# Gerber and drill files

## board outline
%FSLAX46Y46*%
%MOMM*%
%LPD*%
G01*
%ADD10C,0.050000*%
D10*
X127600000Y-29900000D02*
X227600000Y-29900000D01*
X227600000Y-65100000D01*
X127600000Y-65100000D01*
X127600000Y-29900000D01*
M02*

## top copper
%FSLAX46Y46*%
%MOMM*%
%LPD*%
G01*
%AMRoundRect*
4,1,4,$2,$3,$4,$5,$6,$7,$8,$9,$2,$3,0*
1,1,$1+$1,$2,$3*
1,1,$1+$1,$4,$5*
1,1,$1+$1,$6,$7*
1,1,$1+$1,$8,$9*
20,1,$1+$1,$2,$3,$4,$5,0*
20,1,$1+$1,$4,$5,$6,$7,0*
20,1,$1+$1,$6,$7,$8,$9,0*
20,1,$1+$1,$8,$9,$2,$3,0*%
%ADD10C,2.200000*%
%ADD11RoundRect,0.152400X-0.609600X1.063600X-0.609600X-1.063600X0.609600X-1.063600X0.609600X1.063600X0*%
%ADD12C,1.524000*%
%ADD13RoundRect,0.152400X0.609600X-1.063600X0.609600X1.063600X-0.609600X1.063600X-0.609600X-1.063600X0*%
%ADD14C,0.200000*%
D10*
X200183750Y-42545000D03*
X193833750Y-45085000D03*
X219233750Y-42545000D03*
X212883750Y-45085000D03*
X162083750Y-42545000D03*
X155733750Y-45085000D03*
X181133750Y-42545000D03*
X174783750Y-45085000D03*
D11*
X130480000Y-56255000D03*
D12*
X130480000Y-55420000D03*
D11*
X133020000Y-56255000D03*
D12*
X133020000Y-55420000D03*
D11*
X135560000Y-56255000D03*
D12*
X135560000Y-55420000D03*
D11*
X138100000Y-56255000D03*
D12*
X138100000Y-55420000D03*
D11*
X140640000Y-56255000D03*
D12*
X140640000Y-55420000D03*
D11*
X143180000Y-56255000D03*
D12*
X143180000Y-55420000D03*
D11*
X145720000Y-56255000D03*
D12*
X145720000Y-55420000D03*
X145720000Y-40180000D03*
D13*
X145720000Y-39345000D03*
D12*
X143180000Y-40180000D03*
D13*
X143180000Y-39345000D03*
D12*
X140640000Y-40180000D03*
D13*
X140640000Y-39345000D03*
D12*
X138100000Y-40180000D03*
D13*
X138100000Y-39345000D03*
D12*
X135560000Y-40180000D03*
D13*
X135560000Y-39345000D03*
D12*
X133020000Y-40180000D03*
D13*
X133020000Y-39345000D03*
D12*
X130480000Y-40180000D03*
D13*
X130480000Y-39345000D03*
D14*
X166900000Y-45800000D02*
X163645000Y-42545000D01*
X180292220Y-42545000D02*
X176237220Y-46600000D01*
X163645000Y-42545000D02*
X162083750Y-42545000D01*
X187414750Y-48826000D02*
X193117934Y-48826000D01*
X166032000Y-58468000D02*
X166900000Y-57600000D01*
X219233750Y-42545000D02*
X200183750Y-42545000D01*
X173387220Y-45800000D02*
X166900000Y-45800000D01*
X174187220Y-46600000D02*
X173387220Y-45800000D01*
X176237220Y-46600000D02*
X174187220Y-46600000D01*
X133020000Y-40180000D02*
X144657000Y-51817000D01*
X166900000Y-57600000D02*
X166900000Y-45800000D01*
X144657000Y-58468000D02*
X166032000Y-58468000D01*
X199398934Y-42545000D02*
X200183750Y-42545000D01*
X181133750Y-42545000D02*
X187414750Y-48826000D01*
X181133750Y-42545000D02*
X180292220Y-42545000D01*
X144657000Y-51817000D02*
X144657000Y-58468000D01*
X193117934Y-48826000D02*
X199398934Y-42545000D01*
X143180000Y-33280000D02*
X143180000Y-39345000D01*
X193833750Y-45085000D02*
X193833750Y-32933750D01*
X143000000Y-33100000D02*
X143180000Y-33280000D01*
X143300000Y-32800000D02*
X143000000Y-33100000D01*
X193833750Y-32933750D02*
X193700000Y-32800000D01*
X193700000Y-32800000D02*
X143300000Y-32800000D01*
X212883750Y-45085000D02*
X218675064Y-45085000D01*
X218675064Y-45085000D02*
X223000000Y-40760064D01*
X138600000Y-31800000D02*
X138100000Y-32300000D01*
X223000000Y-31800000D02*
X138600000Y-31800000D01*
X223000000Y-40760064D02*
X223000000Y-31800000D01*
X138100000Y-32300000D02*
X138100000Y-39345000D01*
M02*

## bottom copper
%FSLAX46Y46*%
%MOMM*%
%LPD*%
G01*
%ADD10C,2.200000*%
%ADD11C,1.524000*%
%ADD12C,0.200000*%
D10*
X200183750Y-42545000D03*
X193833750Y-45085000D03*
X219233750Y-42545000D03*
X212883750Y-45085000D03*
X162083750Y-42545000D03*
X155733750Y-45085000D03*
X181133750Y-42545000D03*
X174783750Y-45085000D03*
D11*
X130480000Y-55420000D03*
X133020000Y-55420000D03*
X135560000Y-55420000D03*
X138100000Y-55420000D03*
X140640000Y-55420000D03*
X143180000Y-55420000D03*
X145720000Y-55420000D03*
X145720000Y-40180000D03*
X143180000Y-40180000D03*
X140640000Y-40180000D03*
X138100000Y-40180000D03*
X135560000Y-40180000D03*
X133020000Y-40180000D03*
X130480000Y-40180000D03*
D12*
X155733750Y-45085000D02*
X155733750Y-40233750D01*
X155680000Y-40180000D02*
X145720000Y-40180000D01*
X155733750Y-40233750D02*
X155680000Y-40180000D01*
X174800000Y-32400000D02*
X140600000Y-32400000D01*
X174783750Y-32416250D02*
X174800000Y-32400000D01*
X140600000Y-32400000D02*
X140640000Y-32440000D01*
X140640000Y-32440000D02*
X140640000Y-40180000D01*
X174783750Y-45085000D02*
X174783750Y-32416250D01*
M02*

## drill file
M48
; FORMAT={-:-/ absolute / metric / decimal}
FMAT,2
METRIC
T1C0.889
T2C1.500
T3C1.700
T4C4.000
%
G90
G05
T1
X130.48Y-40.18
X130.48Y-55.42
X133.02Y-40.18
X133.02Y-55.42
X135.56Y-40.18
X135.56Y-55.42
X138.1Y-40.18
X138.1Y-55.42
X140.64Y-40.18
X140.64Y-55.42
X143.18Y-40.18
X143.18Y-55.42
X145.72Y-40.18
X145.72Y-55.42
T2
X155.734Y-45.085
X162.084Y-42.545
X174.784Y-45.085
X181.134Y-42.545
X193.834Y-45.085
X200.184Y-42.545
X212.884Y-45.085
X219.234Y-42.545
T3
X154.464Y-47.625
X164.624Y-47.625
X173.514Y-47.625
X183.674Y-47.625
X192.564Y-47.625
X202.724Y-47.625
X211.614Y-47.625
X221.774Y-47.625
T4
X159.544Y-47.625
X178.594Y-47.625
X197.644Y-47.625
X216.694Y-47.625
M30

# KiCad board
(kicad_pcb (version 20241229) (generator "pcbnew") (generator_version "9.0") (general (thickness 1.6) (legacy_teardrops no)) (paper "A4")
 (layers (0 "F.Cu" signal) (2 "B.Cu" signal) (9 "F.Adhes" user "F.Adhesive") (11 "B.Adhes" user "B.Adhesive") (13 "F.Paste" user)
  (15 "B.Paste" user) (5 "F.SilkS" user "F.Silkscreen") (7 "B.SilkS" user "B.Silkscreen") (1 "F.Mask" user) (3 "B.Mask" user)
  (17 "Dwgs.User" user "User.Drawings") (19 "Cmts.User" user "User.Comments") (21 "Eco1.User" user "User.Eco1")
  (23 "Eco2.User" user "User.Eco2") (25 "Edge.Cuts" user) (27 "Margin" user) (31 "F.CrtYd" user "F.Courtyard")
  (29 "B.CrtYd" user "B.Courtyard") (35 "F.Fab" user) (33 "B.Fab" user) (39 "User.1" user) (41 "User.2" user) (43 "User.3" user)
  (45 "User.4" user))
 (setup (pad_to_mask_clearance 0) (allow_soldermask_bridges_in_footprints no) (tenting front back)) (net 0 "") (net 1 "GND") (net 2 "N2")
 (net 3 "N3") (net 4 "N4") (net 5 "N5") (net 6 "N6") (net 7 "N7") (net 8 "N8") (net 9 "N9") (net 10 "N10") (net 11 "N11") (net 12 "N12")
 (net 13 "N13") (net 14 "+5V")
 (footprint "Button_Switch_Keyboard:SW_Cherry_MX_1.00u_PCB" (layer "F.Cu") (at 200.18375 42.545)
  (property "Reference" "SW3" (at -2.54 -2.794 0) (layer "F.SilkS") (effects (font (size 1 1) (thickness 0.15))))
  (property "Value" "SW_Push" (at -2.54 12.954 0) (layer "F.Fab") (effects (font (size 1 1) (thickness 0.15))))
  (pad "" np_thru_hole circle (at -7.62 5.08) (size 1.7 1.7) (drill 1.7) (layers "*.Cu" "*.Mask"))
  (pad "" np_thru_hole circle (at -2.54 5.08) (size 4 4) (drill 4) (layers "*.Cu" "*.Mask"))
  (pad "" np_thru_hole circle (at 2.54 5.08) (size 1.7 1.7) (drill 1.7) (layers "*.Cu" "*.Mask"))
  (pad "1" thru_hole circle (at 0 0) (size 2.2 2.2) (drill 1.5) (layers "*.Cu" "*.Mask") (remove_unused_layers no) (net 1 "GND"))
  (pad "2" thru_hole circle (at -6.35 2.54) (size 2.2 2.2) (drill 1.5) (layers "*.Cu" "*.Mask") (remove_unused_layers no) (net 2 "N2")))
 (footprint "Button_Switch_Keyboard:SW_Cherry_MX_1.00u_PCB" (layer "F.Cu") (at 219.23375 42.545)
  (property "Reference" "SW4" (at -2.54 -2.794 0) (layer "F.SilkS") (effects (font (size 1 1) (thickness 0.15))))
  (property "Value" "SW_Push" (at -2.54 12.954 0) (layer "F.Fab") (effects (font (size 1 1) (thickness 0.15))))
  (pad "" np_thru_hole circle (at -7.62 5.08) (size 1.7 1.7) (drill 1.7) (layers "*.Cu" "*.Mask"))
  (pad "" np_thru_hole circle (at -2.54 5.08) (size 4 4) (drill 4) (layers "*.Cu" "*.Mask"))
  (pad "" np_thru_hole circle (at 2.54 5.08) (size 1.7 1.7) (drill 1.7) (layers "*.Cu" "*.Mask"))
  (pad "1" thru_hole circle (at 0 0) (size 2.2 2.2) (drill 1.5) (layers "*.Cu" "*.Mask") (remove_unused_layers no) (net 1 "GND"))
  (pad "2" thru_hole circle (at -6.35 2.54) (size 2.2 2.2) (drill 1.5) (layers "*.Cu" "*.Mask") (remove_unused_layers no) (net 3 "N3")))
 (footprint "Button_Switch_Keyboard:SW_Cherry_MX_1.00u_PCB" (layer "F.Cu") (at 162.08375 42.545)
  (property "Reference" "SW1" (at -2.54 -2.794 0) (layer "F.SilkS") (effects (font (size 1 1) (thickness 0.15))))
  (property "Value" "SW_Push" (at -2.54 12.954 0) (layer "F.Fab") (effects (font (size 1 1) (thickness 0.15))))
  (pad "" np_thru_hole circle (at -7.62 5.08) (size 1.7 1.7) (drill 1.7) (layers "*.Cu" "*.Mask"))
  (pad "" np_thru_hole circle (at -2.54 5.08) (size 4 4) (drill 4) (layers "*.Cu" "*.Mask"))
  (pad "" np_thru_hole circle (at 2.54 5.08) (size 1.7 1.7) (drill 1.7) (layers "*.Cu" "*.Mask"))
  (pad "1" thru_hole circle (at 0 0) (size 2.2 2.2) (drill 1.5) (layers "*.Cu" "*.Mask") (remove_unused_layers no) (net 1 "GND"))
  (pad "2" thru_hole circle (at -6.35 2.54) (size 2.2 2.2) (drill 1.5) (layers "*.Cu" "*.Mask") (remove_unused_layers no) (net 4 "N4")))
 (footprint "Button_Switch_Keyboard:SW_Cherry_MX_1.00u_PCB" (layer "F.Cu") (at 181.13375 42.545)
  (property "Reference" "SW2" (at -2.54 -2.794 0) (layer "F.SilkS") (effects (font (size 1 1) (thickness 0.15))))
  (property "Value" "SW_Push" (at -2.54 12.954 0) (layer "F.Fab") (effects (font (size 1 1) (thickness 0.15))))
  (pad "" np_thru_hole circle (at -7.62 5.08) (size 1.7 1.7) (drill 1.7) (layers "*.Cu" "*.Mask"))
  (pad "" np_thru_hole circle (at -2.54 5.08) (size 4 4) (drill 4) (layers "*.Cu" "*.Mask"))
  (pad "" np_thru_hole circle (at 2.54 5.08) (size 1.7 1.7) (drill 1.7) (layers "*.Cu" "*.Mask"))
  (pad "1" thru_hole circle (at 0 0) (size 2.2 2.2) (drill 1.5) (layers "*.Cu" "*.Mask") (remove_unused_layers no) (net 1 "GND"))
  (pad "2" thru_hole circle (at -6.35 2.54) (size 2.2 2.2) (drill 1.5) (layers "*.Cu" "*.Mask") (remove_unused_layers no) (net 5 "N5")))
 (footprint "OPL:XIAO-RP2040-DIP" (layer "F.Cu") (at 138.1 47.8 90)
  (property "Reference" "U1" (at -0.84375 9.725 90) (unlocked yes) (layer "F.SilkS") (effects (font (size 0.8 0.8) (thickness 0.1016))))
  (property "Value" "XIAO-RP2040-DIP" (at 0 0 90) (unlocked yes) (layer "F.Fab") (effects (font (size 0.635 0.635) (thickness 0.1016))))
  (pad "1" smd roundrect (at -8.455 -7.62 270) (size 2.432 1.524) (layers "F.Cu" "F.Mask") (roundrect_rratio 0.1) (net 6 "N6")
   (thermal_bridge_angle 45))
  (pad "1" thru_hole circle (at -7.62 -7.62 270) (size 1.524 1.524) (drill 0.889) (layers "*.Cu" "*.Mask") (remove_unused_layers no)
   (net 6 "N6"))
  (pad "2" smd roundrect (at -8.455 -5.08 270) (size 2.432 1.524) (layers "F.Cu" "F.Mask") (roundrect_rratio 0.1) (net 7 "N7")
   (thermal_bridge_angle 45))
  (pad "2" thru_hole circle (at -7.62 -5.08 270) (size 1.524 1.524) (drill 0.889) (layers "*.Cu" "*.Mask") (remove_unused_layers no)
   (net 7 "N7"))
  (pad "3" smd roundrect (at -8.455 -2.54 270) (size 2.432 1.524) (layers "F.Cu" "F.Mask") (roundrect_rratio 0.1) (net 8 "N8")
   (thermal_bridge_angle 45))
  (pad "3" thru_hole circle (at -7.62 -2.54 270) (size 1.524 1.524) (drill 0.889) (layers "*.Cu" "*.Mask") (remove_unused_layers no)
   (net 8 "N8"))
  (pad "4" smd roundrect (at -8.455 0 270) (size 2.432 1.524) (layers "F.Cu" "F.Mask") (roundrect_rratio 0.1) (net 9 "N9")
   (thermal_bridge_angle 45))
  (pad "4" thru_hole circle (at -7.62 0 270) (size 1.524 1.524) (drill 0.889) (layers "*.Cu" "*.Mask") (remove_unused_layers no)
   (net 9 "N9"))
  (pad "5" smd roundrect (at -8.455 2.54 270) (size 2.432 1.524) (layers "F.Cu" "F.Mask") (roundrect_rratio 0.1) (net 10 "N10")
   (thermal_bridge_angle 45))
  (pad "5" thru_hole circle (at -7.62 2.54 270) (size 1.524 1.524) (drill 0.889) (layers "*.Cu" "*.Mask") (remove_unused_layers no)
   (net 10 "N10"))
  (pad "6" smd roundrect (at -8.455 5.08 270) (size 2.432 1.524) (layers "F.Cu" "F.Mask") (roundrect_rratio 0.1) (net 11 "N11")
   (thermal_bridge_angle 45))
  (pad "6" thru_hole circle (at -7.62 5.08 270) (size 1.524 1.524) (drill 0.889) (layers "*.Cu" "*.Mask") (remove_unused_layers no)
   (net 11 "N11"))
  (pad "7" smd roundrect (at -8.455 7.62 270) (size 2.432 1.524) (layers "F.Cu" "F.Mask") (roundrect_rratio 0.1) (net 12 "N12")
   (thermal_bridge_angle 45))
  (pad "7" thru_hole circle (at -7.62 7.62 270) (size 1.524 1.524) (drill 0.889) (layers "*.Cu" "*.Mask") (remove_unused_layers no)
   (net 12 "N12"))
  (pad "8" thru_hole circle (at 7.62 7.62 90) (size 1.524 1.524) (drill 0.889) (layers "*.Cu" "*.Mask") (remove_unused_layers no)
   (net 4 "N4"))
  (pad "8" smd roundrect (at 8.455 7.62 90) (size 2.432 1.524) (layers "F.Cu" "F.Mask") (roundrect_rratio 0.1) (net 4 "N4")
   (thermal_bridge_angle 45))
  (pad "9" thru_hole circle (at 7.62 5.08 90) (size 1.524 1.524) (drill 0.889) (layers "*.Cu" "*.Mask") (remove_unused_layers no)
   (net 2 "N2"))
  (pad "9" smd roundrect (at 8.455 5.08 90) (size 2.432 1.524) (layers "F.Cu" "F.Mask") (roundrect_rratio 0.1) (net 2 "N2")
   (thermal_bridge_angle 45))
  (pad "10" thru_hole circle (at 7.62 2.54 90) (size 1.524 1.524) (drill 0.889) (layers "*.Cu" "*.Mask") (remove_unused_layers no)
   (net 5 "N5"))
  (pad "10" smd roundrect (at 8.455 2.54 90) (size 2.432 1.524) (layers "F.Cu" "F.Mask") (roundrect_rratio 0.1) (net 5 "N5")
   (thermal_bridge_angle 45))
  (pad "11" thru_hole circle (at 7.62 0 90) (size 1.524 1.524) (drill 0.889) (layers "*.Cu" "*.Mask") (remove_unused_layers no) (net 3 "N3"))
  (pad "11" smd roundrect (at 8.455 0 90) (size 2.432 1.524) (layers "F.Cu" "F.Mask") (roundrect_rratio 0.1) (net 3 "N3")
   (thermal_bridge_angle 45))
  (pad "12" thru_hole circle (at 7.62 -2.54 90) (size 1.524 1.524) (drill 0.889) (layers "*.Cu" "*.Mask") (remove_unused_layers no)
   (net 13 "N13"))
  (pad "12" smd roundrect (at 8.455 -2.54 90) (size 2.432 1.524) (layers "F.Cu" "F.Mask") (roundrect_rratio 0.1) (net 13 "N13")
   (thermal_bridge_angle 45))
  (pad "13" thru_hole circle (at 7.62 -5.08 90) (size 1.524 1.524) (drill 0.889) (layers "*.Cu" "*.Mask") (remove_unused_layers no)
   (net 1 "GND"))
  (pad "13" smd roundrect (at 8.455 -5.08 90) (size 2.432 1.524) (layers "F.Cu" "F.Mask") (roundrect_rratio 0.1) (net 1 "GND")
   (thermal_bridge_angle 45))
  (pad "14" thru_hole circle (at 7.62 -7.62 90) (size 1.524 1.524) (drill 0.889) (layers "*.Cu" "*.Mask") (remove_unused_layers no)
   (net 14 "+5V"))
  (pad "14" smd roundrect (at 8.455 -7.62 90) (size 2.432 1.524) (layers "F.Cu" "F.Mask") (roundrect_rratio 0.1) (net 14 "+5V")
   (thermal_bridge_angle 45)))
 (gr_rect (start 127.6 29.9) (end 227.6 65.1) (stroke (width 0.05) (type default)) (fill no) (layer "Edge.Cuts"))
 (segment (start 166.9 45.8) (end 163.645 42.545) (width 0.2) (layer "F.Cu") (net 1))
 (segment (start 180.29222 42.545) (end 176.23722 46.6) (width 0.2) (layer "F.Cu") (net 1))
 (segment (start 163.645 42.545) (end 162.08375 42.545) (width 0.2) (layer "F.Cu") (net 1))
 (segment (start 187.41475 48.826) (end 193.117934 48.826) (width 0.2) (layer "F.Cu") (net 1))
 (segment (start 166.032 58.468) (end 166.9 57.6) (width 0.2) (layer "F.Cu") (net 1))
 (segment (start 219.23375 42.545) (end 200.18375 42.545) (width 0.2) (layer "F.Cu") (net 1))
 (segment (start 173.38722 45.8) (end 166.9 45.8) (width 0.2) (layer "F.Cu") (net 1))
 (segment (start 174.18722 46.6) (end 173.38722 45.8) (width 0.2) (layer "F.Cu") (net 1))
 (segment (start 176.23722 46.6) (end 174.18722 46.6) (width 0.2) (layer "F.Cu") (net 1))
 (segment (start 133.02 40.18) (end 144.657 51.817) (width 0.2) (layer "F.Cu") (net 1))
 (segment (start 166.9 57.6) (end 166.9 45.8) (width 0.2) (layer "F.Cu") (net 1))
 (segment (start 144.657 58.468) (end 166.032 58.468) (width 0.2) (layer "F.Cu") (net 1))
 (segment (start 199.398934 42.545) (end 200.18375 42.545) (width 0.2) (layer "F.Cu") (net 1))
 (segment (start 181.13375 42.545) (end 187.41475 48.826) (width 0.2) (layer "F.Cu") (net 1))
 (segment (start 181.13375 42.545) (end 180.29222 42.545) (width 0.2) (layer "F.Cu") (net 1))
 (segment (start 144.657 51.817) (end 144.657 58.468) (width 0.2) (layer "F.Cu") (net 1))
 (segment (start 193.117934 48.826) (end 199.398934 42.545) (width 0.2) (layer "F.Cu") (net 1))
 (segment (start 155.73375 45.085) (end 155.73375 40.23375) (width 0.2) (layer "B.Cu") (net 4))
 (segment (start 155.68 40.18) (end 145.72 40.18) (width 0.2) (layer "B.Cu") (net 4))
 (segment (start 155.73375 40.23375) (end 155.68 40.18) (width 0.2) (layer "B.Cu") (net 4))
 (segment (start 174.8 32.4) (end 140.6 32.4) (width 0.2) (layer "B.Cu") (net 5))
 (segment (start 174.78375 32.41625) (end 174.8 32.4) (width 0.2) (layer "B.Cu") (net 5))
 (segment (start 140.6 32.4) (end 140.64 32.44) (width 0.2) (layer "B.Cu") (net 5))
 (segment (start 140.64 32.44) (end 140.64 40.18) (width 0.2) (layer "B.Cu") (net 5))
 (segment (start 174.78375 45.085) (end 174.78375 32.41625) (width 0.2) (layer "B.Cu") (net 5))
 (segment (start 143.18 33.28) (end 143.18 39.345) (width 0.2) (layer "F.Cu") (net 2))
 (segment (start 193.83375 45.085) (end 193.83375 32.93375) (width 0.2) (layer "F.Cu") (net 2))
 (segment (start 143 33.1) (end 143.18 33.28) (width 0.2) (layer "F.Cu") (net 2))
 (segment (start 143.3 32.8) (end 143 33.1) (width 0.2) (layer "F.Cu") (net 2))
 (segment (start 193.83375 32.93375) (end 193.7 32.8) (width 0.2) (layer "F.Cu") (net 2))
 (segment (start 193.7 32.8) (end 143.3 32.8) (width 0.2) (layer "F.Cu") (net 2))
 (segment (start 212.88375 45.085) (end 218.675064 45.085) (width 0.2) (layer "F.Cu") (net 3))
 (segment (start 218.675064 45.085) (end 223 40.760064) (width 0.2) (layer "F.Cu") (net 3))
 (segment (start 138.6 31.8) (end 138.1 32.3) (width 0.2) (layer "F.Cu") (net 3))
 (segment (start 223 31.8) (end 138.6 31.8) (width 0.2) (layer "F.Cu") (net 3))
 (segment (start 223 40.760064) (end 223 31.8) (width 0.2) (layer "F.Cu") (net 3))
 (segment (start 138.1 32.3) (end 138.1 39.345) (width 0.2) (layer "F.Cu") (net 3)))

